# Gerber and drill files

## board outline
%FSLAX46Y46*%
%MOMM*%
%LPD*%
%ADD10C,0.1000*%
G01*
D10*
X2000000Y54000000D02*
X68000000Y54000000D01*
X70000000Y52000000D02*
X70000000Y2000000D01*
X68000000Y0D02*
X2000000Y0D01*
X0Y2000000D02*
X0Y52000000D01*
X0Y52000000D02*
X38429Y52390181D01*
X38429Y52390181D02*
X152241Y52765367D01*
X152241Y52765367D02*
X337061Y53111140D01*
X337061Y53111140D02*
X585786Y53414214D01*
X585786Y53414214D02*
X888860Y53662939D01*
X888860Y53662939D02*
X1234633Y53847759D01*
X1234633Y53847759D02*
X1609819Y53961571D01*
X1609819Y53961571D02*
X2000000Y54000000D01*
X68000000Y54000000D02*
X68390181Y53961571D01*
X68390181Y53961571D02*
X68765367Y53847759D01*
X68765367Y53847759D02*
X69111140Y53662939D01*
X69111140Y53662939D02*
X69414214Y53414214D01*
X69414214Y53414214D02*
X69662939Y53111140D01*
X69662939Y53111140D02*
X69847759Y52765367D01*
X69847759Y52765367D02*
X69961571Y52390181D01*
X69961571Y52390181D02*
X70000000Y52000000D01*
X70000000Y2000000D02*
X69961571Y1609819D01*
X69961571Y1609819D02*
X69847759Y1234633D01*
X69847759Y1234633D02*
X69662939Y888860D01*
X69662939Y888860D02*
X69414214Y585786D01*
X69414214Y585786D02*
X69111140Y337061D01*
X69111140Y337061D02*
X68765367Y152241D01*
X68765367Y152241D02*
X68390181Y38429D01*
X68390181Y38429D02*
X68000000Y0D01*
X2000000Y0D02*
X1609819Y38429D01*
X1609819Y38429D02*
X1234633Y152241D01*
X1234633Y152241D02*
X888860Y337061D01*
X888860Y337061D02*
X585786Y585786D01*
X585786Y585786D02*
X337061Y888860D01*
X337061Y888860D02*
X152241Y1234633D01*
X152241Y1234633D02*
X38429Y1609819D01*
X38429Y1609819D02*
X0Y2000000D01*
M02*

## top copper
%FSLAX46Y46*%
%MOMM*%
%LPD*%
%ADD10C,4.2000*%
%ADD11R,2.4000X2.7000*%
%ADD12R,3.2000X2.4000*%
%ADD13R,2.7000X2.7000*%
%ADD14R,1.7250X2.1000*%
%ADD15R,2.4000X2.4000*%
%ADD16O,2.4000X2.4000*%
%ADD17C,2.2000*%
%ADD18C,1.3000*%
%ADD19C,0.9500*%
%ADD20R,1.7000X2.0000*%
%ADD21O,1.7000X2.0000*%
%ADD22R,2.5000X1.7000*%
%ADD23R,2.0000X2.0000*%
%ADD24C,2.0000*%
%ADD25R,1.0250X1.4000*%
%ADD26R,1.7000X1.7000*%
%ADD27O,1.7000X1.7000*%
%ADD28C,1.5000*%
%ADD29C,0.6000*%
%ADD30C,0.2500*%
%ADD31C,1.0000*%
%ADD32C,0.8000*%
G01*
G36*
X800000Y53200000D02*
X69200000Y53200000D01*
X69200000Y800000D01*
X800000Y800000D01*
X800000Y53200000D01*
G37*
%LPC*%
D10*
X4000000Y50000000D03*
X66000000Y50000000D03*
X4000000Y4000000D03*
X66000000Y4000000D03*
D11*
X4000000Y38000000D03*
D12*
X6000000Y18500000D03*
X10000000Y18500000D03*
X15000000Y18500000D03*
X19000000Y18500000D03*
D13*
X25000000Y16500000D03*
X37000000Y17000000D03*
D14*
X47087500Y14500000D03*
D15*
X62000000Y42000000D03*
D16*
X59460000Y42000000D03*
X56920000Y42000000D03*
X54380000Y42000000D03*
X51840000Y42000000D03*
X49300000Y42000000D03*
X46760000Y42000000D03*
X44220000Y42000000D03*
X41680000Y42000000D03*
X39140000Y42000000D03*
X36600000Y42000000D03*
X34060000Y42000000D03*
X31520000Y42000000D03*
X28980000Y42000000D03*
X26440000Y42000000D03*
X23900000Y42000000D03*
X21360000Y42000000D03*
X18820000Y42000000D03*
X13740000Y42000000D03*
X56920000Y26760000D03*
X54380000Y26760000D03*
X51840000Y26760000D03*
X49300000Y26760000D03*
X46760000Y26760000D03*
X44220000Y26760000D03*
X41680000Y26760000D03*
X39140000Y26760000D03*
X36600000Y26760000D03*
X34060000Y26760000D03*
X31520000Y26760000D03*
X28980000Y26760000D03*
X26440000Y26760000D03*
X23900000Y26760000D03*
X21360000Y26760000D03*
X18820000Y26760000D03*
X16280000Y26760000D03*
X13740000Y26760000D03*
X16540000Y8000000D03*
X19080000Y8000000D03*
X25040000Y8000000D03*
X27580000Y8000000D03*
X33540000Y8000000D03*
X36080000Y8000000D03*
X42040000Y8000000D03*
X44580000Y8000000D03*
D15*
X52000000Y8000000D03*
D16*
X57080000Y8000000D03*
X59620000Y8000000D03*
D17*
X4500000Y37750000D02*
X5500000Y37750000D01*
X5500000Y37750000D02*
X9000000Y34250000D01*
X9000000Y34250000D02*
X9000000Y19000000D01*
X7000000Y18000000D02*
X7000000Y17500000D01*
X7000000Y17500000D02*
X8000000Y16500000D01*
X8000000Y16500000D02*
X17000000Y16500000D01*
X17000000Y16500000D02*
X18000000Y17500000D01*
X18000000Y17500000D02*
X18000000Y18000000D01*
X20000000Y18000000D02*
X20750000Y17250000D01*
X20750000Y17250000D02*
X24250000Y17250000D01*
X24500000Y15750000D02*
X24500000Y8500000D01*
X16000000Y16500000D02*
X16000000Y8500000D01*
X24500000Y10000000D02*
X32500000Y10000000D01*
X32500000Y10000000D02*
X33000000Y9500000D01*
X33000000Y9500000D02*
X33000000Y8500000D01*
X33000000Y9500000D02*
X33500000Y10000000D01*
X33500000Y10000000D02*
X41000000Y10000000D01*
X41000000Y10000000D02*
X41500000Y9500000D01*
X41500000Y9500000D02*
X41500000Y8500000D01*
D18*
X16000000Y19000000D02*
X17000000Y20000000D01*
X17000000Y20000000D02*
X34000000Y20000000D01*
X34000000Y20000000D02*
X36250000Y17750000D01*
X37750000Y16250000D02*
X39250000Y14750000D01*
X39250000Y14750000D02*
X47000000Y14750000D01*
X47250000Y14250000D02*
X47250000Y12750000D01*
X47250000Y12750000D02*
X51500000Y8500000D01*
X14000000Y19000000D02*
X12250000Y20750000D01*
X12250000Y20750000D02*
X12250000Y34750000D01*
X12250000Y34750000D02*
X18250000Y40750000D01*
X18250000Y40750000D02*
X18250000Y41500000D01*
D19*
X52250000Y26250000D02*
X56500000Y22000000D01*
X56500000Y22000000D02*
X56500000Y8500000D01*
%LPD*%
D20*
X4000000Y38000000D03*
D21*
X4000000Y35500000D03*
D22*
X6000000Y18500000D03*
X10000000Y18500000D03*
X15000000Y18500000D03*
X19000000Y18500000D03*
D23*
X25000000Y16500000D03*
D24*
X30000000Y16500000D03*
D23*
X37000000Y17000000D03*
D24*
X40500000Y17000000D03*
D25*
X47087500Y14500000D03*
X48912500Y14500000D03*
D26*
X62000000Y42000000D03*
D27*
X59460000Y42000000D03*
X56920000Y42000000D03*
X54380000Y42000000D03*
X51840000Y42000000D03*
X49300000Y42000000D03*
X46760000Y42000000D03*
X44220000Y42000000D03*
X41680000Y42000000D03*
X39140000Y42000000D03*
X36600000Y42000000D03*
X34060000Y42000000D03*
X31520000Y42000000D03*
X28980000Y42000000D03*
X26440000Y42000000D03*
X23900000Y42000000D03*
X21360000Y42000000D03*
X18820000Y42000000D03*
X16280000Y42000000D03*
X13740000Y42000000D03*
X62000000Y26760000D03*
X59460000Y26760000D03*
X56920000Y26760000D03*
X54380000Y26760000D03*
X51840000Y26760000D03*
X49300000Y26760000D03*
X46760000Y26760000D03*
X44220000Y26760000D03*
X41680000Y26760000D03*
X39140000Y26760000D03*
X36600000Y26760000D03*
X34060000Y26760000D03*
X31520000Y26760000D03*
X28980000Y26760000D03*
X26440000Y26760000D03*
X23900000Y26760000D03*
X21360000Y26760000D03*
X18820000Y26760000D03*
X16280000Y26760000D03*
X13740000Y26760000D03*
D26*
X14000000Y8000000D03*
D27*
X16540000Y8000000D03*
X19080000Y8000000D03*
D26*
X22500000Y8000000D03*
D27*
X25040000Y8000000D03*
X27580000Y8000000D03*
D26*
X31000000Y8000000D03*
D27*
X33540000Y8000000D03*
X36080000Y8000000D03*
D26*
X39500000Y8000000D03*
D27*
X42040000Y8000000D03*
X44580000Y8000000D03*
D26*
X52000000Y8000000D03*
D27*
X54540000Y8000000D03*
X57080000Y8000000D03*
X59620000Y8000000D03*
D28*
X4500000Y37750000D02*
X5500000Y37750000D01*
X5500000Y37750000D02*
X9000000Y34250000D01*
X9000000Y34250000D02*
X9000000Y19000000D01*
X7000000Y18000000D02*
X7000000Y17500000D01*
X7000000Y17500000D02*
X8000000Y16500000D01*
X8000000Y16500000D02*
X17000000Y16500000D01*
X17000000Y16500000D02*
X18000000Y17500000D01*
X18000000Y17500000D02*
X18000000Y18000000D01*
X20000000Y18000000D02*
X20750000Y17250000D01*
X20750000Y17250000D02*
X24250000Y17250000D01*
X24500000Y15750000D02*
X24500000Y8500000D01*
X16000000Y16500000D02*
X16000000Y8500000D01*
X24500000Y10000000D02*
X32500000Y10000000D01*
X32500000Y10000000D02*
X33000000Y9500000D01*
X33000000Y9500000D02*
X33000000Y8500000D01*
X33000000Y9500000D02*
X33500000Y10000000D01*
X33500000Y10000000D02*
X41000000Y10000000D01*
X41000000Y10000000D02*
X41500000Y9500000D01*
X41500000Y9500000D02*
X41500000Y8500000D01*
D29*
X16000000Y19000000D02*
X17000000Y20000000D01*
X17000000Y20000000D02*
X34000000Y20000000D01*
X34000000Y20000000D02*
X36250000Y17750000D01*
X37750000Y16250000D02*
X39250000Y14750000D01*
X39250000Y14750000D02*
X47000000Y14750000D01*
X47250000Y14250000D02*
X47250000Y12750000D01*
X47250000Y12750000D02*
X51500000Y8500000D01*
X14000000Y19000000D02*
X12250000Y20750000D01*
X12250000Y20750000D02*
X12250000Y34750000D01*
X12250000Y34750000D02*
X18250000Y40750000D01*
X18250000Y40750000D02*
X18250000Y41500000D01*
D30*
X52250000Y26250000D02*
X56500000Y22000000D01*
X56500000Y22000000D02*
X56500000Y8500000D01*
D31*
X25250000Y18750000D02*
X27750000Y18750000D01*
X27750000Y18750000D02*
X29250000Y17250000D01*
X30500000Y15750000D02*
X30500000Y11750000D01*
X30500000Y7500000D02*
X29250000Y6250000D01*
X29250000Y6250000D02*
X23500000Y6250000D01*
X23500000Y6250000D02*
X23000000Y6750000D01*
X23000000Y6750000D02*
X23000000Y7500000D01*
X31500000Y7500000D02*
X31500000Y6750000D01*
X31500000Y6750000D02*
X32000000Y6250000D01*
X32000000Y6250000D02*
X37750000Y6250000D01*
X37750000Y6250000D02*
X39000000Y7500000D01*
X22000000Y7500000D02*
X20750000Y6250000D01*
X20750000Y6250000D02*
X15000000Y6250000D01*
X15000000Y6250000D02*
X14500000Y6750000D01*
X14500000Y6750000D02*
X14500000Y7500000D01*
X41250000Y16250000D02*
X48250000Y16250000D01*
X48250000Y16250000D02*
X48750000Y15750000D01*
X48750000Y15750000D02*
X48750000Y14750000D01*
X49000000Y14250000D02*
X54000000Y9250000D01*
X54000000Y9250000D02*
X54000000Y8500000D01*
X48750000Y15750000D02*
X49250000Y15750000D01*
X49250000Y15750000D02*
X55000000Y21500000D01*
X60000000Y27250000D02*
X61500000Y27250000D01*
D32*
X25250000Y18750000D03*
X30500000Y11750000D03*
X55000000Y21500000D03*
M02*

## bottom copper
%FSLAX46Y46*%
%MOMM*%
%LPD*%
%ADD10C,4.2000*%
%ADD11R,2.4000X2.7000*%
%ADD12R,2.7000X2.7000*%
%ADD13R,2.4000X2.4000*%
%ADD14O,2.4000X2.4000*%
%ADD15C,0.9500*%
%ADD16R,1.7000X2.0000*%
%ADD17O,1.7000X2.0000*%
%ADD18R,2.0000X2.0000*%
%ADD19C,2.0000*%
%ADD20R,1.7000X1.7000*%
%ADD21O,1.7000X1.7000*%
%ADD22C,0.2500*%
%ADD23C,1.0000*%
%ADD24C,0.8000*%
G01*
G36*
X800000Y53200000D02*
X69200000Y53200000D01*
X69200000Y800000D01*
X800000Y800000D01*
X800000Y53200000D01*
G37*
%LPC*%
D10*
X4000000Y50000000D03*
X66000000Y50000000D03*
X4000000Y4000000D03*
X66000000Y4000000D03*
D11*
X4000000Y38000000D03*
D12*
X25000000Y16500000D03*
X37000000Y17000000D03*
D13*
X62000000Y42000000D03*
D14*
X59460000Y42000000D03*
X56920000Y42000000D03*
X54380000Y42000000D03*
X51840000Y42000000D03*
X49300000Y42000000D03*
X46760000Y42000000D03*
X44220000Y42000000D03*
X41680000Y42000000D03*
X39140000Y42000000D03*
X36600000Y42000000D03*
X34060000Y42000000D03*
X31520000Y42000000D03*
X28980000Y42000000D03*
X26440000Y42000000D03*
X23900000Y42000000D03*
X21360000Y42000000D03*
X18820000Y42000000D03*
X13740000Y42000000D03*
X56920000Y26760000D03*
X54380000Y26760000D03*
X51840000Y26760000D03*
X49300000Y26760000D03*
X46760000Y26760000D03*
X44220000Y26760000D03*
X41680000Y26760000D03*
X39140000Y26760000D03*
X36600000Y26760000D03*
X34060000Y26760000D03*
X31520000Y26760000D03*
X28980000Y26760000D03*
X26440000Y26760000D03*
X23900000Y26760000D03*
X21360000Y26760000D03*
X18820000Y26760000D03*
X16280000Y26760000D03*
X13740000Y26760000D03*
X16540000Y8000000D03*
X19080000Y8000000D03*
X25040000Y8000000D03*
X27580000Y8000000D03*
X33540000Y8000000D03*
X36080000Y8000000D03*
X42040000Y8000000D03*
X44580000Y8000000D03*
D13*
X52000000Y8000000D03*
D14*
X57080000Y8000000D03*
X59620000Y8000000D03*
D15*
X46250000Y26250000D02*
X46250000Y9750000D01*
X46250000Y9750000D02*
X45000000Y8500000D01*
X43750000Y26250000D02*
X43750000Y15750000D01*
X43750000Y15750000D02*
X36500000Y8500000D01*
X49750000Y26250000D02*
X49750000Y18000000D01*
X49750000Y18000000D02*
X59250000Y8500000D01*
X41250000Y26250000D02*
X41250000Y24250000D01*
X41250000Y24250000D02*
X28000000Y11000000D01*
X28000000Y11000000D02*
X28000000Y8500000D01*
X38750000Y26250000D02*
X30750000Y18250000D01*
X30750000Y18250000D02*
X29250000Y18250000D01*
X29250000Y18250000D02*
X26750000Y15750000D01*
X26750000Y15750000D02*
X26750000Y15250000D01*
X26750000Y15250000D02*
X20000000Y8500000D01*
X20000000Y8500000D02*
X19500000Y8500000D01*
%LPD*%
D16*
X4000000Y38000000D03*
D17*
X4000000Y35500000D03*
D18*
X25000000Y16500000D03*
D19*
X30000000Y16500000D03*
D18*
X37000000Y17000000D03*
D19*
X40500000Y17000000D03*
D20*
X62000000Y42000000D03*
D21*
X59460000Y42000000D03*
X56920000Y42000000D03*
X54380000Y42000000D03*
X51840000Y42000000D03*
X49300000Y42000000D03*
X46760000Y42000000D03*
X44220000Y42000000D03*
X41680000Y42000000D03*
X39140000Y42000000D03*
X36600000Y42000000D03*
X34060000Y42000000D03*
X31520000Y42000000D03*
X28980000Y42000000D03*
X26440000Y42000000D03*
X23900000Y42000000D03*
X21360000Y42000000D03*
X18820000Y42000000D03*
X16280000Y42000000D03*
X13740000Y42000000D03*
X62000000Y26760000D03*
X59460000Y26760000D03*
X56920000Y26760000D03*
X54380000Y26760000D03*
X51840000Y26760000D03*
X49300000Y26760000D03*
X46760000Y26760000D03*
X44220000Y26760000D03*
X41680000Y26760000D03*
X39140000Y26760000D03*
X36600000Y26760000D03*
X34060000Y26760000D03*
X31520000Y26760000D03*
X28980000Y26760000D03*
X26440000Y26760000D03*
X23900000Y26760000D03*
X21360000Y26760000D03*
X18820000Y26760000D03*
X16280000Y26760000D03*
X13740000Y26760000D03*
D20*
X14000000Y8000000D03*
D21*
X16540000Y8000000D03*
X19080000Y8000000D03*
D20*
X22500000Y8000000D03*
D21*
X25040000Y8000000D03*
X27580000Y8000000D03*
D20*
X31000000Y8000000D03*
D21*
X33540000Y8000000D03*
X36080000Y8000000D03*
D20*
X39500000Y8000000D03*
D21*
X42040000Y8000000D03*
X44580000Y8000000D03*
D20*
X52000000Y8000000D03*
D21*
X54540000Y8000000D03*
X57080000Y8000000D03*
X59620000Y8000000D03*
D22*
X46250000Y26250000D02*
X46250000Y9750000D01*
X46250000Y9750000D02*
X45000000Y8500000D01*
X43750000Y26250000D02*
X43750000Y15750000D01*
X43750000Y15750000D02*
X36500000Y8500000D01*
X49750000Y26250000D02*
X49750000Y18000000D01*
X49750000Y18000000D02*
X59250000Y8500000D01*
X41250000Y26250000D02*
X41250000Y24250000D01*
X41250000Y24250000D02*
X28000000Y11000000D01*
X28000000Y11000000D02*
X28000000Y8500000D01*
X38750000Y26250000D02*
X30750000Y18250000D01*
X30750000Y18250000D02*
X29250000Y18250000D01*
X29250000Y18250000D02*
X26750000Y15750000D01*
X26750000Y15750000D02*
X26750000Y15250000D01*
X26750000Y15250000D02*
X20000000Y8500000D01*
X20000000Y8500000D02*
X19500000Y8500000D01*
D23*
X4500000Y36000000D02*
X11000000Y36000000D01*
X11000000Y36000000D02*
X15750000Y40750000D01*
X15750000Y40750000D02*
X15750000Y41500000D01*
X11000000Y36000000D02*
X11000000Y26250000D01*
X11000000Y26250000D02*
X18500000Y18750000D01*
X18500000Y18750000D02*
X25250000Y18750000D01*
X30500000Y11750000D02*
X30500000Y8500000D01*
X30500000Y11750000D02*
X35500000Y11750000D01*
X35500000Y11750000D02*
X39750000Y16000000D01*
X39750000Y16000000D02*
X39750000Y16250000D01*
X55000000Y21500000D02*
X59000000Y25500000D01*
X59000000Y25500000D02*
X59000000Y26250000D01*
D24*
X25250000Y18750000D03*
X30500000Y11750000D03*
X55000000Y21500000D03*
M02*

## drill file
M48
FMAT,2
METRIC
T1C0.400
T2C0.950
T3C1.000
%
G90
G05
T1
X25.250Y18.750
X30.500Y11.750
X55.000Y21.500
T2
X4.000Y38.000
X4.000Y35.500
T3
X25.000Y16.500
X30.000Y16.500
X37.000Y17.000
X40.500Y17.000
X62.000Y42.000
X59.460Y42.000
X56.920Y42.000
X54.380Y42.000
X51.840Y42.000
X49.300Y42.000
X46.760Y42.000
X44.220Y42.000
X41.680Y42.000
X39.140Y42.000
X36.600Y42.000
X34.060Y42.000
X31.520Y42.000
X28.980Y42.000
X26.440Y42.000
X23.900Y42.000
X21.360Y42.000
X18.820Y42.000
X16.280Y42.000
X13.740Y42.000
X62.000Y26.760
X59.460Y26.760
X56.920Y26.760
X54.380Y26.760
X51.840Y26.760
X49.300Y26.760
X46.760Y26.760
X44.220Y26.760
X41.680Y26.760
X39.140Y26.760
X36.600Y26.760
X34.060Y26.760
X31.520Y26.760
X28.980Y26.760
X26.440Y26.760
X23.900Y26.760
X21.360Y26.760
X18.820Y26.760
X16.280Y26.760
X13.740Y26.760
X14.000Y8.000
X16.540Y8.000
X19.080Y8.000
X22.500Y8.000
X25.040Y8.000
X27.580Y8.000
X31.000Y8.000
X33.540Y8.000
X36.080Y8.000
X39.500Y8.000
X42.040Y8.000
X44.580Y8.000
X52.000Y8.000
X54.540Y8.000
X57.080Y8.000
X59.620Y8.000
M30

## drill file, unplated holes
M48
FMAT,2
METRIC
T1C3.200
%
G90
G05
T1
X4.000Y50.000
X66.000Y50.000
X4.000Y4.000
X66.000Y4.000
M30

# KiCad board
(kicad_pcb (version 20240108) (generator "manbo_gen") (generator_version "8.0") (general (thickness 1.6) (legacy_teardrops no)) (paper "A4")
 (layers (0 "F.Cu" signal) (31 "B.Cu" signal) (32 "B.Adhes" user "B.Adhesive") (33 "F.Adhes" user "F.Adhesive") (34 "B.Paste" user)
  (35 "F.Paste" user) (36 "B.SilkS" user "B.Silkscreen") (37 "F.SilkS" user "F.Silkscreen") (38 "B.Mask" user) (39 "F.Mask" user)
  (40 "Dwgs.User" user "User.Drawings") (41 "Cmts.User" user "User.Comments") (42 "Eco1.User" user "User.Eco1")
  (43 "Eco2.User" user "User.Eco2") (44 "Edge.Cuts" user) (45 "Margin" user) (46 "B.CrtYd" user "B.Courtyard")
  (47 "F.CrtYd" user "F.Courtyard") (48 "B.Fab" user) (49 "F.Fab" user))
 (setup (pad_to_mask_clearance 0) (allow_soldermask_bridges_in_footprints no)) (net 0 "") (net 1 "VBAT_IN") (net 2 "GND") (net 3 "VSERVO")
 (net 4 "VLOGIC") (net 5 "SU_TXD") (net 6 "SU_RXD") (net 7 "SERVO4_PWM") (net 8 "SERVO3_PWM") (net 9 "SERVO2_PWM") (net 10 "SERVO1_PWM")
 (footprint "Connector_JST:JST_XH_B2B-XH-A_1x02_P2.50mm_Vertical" (layer "F.Cu") (at 4 16 0)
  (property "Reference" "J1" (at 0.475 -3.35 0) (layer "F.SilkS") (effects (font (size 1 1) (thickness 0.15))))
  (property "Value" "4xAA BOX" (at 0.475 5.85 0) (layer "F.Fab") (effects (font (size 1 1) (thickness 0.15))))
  (pad "1" thru_hole roundrect (at 0 0 0) (size 1.7 2) (drill 0.95) (layers "*.Cu" "*.Mask") (roundrect_rratio 0.25) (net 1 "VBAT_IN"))
  (pad "2" thru_hole oval (at 0 2.5 0) (size 1.7 2) (drill 0.95) (layers "*.Cu" "*.Mask") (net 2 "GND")))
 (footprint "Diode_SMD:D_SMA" (layer "F.Cu") (at 8 35.5 0)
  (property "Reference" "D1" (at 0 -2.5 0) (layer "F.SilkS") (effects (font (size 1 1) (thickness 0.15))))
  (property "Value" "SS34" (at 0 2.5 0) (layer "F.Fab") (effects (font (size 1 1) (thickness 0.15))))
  (pad "1" smd rect (at -2 0 0) (size 2.5 1.7) (layers "F.Cu" "F.Paste" "F.Mask") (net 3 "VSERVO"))
  (pad "2" smd rect (at 2 0 0) (size 2.5 1.7) (layers "F.Cu" "F.Paste" "F.Mask") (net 1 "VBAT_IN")))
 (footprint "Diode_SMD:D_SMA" (layer "F.Cu") (at 17 35.5 0)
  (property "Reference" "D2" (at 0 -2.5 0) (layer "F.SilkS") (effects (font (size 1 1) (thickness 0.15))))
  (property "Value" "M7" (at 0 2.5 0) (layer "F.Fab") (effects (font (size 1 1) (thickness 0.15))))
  (pad "1" smd rect (at -2 0 0) (size 2.5 1.7) (layers "F.Cu" "F.Paste" "F.Mask") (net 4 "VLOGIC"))
  (pad "2" smd rect (at 2 0 0) (size 2.5 1.7) (layers "F.Cu" "F.Paste" "F.Mask") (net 3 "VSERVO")))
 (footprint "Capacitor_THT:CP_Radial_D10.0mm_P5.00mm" (layer "F.Cu") (at 25 37.5 0)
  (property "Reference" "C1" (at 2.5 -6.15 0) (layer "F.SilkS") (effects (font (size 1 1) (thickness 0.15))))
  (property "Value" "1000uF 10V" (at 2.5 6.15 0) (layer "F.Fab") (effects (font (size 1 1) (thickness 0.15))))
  (pad "1" thru_hole rect (at 0 0 0) (size 2 2) (drill 1) (layers "*.Cu" "*.Mask") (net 3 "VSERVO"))
  (pad "2" thru_hole circle (at 5 0 0) (size 2 2) (drill 1) (layers "*.Cu" "*.Mask") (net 2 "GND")))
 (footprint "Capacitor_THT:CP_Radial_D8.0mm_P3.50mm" (layer "F.Cu") (at 37 37 0)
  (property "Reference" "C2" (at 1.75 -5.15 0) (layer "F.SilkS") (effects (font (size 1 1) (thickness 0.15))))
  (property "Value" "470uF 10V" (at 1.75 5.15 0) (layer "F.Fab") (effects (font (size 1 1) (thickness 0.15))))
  (pad "1" thru_hole rect (at 0 0 0) (size 2 2) (drill 1) (layers "*.Cu" "*.Mask") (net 4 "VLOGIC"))
  (pad "2" thru_hole circle (at 3.5 0 0) (size 2 2) (drill 1) (layers "*.Cu" "*.Mask") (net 2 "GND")))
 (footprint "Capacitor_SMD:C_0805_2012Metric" (layer "F.Cu") (at 48 39.5 0)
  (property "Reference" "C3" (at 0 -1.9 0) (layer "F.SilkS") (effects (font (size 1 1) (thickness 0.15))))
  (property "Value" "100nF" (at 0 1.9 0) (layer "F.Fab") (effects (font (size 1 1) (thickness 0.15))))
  (pad "1" smd roundrect (at -0.9125 0 0) (size 1.025 1.4) (layers "F.Cu" "F.Paste" "F.Mask") (roundrect_rratio 0.25) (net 4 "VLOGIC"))
  (pad "2" smd roundrect (at 0.9125 0 0) (size 1.025 1.4) (layers "F.Cu" "F.Paste" "F.Mask") (roundrect_rratio 0.25) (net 2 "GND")))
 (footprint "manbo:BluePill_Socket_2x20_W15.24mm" (layer "F.Cu") (at 62 12 270)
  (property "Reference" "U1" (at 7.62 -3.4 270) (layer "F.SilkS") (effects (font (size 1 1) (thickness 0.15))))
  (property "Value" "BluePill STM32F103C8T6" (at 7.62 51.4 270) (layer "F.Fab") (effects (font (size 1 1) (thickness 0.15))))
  (pad "1" thru_hole rect (at 0 0 270) (size 1.7 1.7) (drill 1) (layers "*.Cu" "*.Mask"))
  (pad "2" thru_hole oval (at 0 2.54 270) (size 1.7 1.7) (drill 1) (layers "*.Cu" "*.Mask"))
  (pad "3" thru_hole oval (at 0 5.08 270) (size 1.7 1.7) (drill 1) (layers "*.Cu" "*.Mask"))
  (pad "4" thru_hole oval (at 0 7.62 270) (size 1.7 1.7) (drill 1) (layers "*.Cu" "*.Mask"))
  (pad "5" thru_hole oval (at 0 10.16 270) (size 1.7 1.7) (drill 1) (layers "*.Cu" "*.Mask"))
  (pad "6" thru_hole oval (at 0 12.7 270) (size 1.7 1.7) (drill 1) (layers "*.Cu" "*.Mask"))
  (pad "7" thru_hole oval (at 0 15.24 270) (size 1.7 1.7) (drill 1) (layers "*.Cu" "*.Mask"))
  (pad "8" thru_hole oval (at 0 17.78 270) (size 1.7 1.7) (drill 1) (layers "*.Cu" "*.Mask"))
  (pad "9" thru_hole oval (at 0 20.32 270) (size 1.7 1.7) (drill 1) (layers "*.Cu" "*.Mask"))
  (pad "10" thru_hole oval (at 0 22.86 270) (size 1.7 1.7) (drill 1) (layers "*.Cu" "*.Mask"))
  (pad "11" thru_hole oval (at 0 25.4 270) (size 1.7 1.7) (drill 1) (layers "*.Cu" "*.Mask"))
  (pad "12" thru_hole oval (at 0 27.94 270) (size 1.7 1.7) (drill 1) (layers "*.Cu" "*.Mask"))
  (pad "13" thru_hole oval (at 0 30.48 270) (size 1.7 1.7) (drill 1) (layers "*.Cu" "*.Mask"))
  (pad "14" thru_hole oval (at 0 33.02 270) (size 1.7 1.7) (drill 1) (layers "*.Cu" "*.Mask"))
  (pad "15" thru_hole oval (at 0 35.56 270) (size 1.7 1.7) (drill 1) (layers "*.Cu" "*.Mask"))
  (pad "16" thru_hole oval (at 0 38.1 270) (size 1.7 1.7) (drill 1) (layers "*.Cu" "*.Mask"))
  (pad "17" thru_hole oval (at 0 40.64 270) (size 1.7 1.7) (drill 1) (layers "*.Cu" "*.Mask"))
  (pad "18" thru_hole oval (at 0 43.18 270) (size 1.7 1.7) (drill 1) (layers "*.Cu" "*.Mask") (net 4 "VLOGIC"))
  (pad "19" thru_hole oval (at 0 45.72 270) (size 1.7 1.7) (drill 1) (layers "*.Cu" "*.Mask") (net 2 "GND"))
  (pad "20" thru_hole oval (at 0 48.26 270) (size 1.7 1.7) (drill 1) (layers "*.Cu" "*.Mask"))
  (pad "21" thru_hole oval (at 15.24 0 270) (size 1.7 1.7) (drill 1) (layers "*.Cu" "*.Mask") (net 2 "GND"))
  (pad "22" thru_hole oval (at 15.24 2.54 270) (size 1.7 1.7) (drill 1) (layers "*.Cu" "*.Mask") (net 2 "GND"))
  (pad "23" thru_hole oval (at 15.24 5.08 270) (size 1.7 1.7) (drill 1) (layers "*.Cu" "*.Mask"))
  (pad "24" thru_hole oval (at 15.24 7.62 270) (size 1.7 1.7) (drill 1) (layers "*.Cu" "*.Mask"))
  (pad "25" thru_hole oval (at 15.24 10.16 270) (size 1.7 1.7) (drill 1) (layers "*.Cu" "*.Mask") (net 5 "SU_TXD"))
  (pad "26" thru_hole oval (at 15.24 12.7 270) (size 1.7 1.7) (drill 1) (layers "*.Cu" "*.Mask") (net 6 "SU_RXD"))
  (pad "27" thru_hole oval (at 15.24 15.24 270) (size 1.7 1.7) (drill 1) (layers "*.Cu" "*.Mask") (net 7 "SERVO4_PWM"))
  (pad "28" thru_hole oval (at 15.24 17.78 270) (size 1.7 1.7) (drill 1) (layers "*.Cu" "*.Mask") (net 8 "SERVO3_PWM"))
  (pad "29" thru_hole oval (at 15.24 20.32 270) (size 1.7 1.7) (drill 1) (layers "*.Cu" "*.Mask") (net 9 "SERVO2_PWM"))
  (pad "30" thru_hole oval (at 15.24 22.86 270) (size 1.7 1.7) (drill 1) (layers "*.Cu" "*.Mask") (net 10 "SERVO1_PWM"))
  (pad "31" thru_hole oval (at 15.24 25.4 270) (size 1.7 1.7) (drill 1) (layers "*.Cu" "*.Mask"))
  (pad "32" thru_hole oval (at 15.24 27.94 270) (size 1.7 1.7) (drill 1) (layers "*.Cu" "*.Mask"))
  (pad "33" thru_hole oval (at 15.24 30.48 270) (size 1.7 1.7) (drill 1) (layers "*.Cu" "*.Mask"))
  (pad "34" thru_hole oval (at 15.24 33.02 270) (size 1.7 1.7) (drill 1) (layers "*.Cu" "*.Mask"))
  (pad "35" thru_hole oval (at 15.24 35.56 270) (size 1.7 1.7) (drill 1) (layers "*.Cu" "*.Mask"))
  (pad "36" thru_hole oval (at 15.24 38.1 270) (size 1.7 1.7) (drill 1) (layers "*.Cu" "*.Mask"))
  (pad "37" thru_hole oval (at 15.24 40.64 270) (size 1.7 1.7) (drill 1) (layers "*.Cu" "*.Mask"))
  (pad "38" thru_hole oval (at 15.24 43.18 270) (size 1.7 1.7) (drill 1) (layers "*.Cu" "*.Mask"))
  (pad "39" thru_hole oval (at 15.24 45.72 270) (size 1.7 1.7) (drill 1) (layers "*.Cu" "*.Mask"))
  (pad "40" thru_hole oval (at 15.24 48.26 270) (size 1.7 1.7) (drill 1) (layers "*.Cu" "*.Mask")))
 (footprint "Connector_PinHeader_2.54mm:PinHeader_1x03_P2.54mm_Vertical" (layer "F.Cu") (at 14 46 90)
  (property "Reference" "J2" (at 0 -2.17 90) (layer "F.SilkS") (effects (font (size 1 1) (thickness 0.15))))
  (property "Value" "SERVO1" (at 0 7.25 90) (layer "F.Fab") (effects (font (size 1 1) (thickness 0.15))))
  (pad "1" thru_hole rect (at 0 0 90) (size 1.7 1.7) (drill 1) (layers "*.Cu" "*.Mask") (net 2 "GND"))
  (pad "2" thru_hole oval (at 0 2.54 90) (size 1.7 1.7) (drill 1) (layers "*.Cu" "*.Mask") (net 3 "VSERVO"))
  (pad "3" thru_hole oval (at 0 5.08 90) (size 1.7 1.7) (drill 1) (layers "*.Cu" "*.Mask") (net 10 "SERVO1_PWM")))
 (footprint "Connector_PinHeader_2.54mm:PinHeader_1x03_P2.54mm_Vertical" (layer "F.Cu") (at 22.5 46 90)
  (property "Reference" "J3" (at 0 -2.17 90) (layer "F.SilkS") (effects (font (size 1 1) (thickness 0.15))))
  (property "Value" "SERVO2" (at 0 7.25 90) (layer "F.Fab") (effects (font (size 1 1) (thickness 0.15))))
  (pad "1" thru_hole rect (at 0 0 90) (size 1.7 1.7) (drill 1) (layers "*.Cu" "*.Mask") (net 2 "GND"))
  (pad "2" thru_hole oval (at 0 2.54 90) (size 1.7 1.7) (drill 1) (layers "*.Cu" "*.Mask") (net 3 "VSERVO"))
  (pad "3" thru_hole oval (at 0 5.08 90) (size 1.7 1.7) (drill 1) (layers "*.Cu" "*.Mask") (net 9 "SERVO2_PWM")))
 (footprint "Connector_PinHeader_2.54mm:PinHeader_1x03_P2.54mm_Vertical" (layer "F.Cu") (at 31 46 90)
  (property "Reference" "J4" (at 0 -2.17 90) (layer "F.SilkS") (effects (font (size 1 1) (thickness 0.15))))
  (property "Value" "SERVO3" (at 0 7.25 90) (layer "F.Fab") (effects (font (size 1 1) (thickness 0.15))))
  (pad "1" thru_hole rect (at 0 0 90) (size 1.7 1.7) (drill 1) (layers "*.Cu" "*.Mask") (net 2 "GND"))
  (pad "2" thru_hole oval (at 0 2.54 90) (size 1.7 1.7) (drill 1) (layers "*.Cu" "*.Mask") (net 3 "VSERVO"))
  (pad "3" thru_hole oval (at 0 5.08 90) (size 1.7 1.7) (drill 1) (layers "*.Cu" "*.Mask") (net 8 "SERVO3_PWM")))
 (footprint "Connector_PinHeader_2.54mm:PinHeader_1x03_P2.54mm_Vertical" (layer "F.Cu") (at 39.5 46 90)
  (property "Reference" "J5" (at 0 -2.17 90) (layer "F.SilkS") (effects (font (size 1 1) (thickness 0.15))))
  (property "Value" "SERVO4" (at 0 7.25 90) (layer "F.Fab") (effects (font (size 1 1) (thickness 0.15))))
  (pad "1" thru_hole rect (at 0 0 90) (size 1.7 1.7) (drill 1) (layers "*.Cu" "*.Mask") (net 2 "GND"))
  (pad "2" thru_hole oval (at 0 2.54 90) (size 1.7 1.7) (drill 1) (layers "*.Cu" "*.Mask") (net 3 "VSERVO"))
  (pad "3" thru_hole oval (at 0 5.08 90) (size 1.7 1.7) (drill 1) (layers "*.Cu" "*.Mask") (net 7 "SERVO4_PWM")))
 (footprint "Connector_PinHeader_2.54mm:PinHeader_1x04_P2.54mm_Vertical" (layer "F.Cu") (at 52 46 90)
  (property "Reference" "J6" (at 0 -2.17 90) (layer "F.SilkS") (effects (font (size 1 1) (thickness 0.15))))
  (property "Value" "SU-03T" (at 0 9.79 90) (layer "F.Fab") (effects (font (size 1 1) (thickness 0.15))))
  (pad "1" thru_hole rect (at 0 0 90) (size 1.7 1.7) (drill 1) (layers "*.Cu" "*.Mask") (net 4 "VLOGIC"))
  (pad "2" thru_hole oval (at 0 2.54 90) (size 1.7 1.7) (drill 1) (layers "*.Cu" "*.Mask") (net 2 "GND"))
  (pad "3" thru_hole oval (at 0 5.08 90) (size 1.7 1.7) (drill 1) (layers "*.Cu" "*.Mask") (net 5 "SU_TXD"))
  (pad "4" thru_hole oval (at 0 7.62 90) (size 1.7 1.7) (drill 1) (layers "*.Cu" "*.Mask") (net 6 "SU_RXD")))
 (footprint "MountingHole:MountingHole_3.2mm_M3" (layer "F.Cu") (at 4 4 0)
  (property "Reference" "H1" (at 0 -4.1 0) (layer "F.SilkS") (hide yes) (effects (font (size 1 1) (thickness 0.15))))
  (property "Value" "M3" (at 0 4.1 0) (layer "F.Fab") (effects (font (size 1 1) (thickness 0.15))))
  (pad "" np_thru_hole circle (at 0 0 0) (size 3.2 3.2) (drill 3.2) (layers "*.Cu" "*.Mask")))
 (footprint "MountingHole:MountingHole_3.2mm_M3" (layer "F.Cu") (at 66 4 0)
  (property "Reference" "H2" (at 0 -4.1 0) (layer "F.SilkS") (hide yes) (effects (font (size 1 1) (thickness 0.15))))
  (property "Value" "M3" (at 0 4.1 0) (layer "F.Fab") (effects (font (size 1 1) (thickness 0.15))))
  (pad "" np_thru_hole circle (at 0 0 0) (size 3.2 3.2) (drill 3.2) (layers "*.Cu" "*.Mask")))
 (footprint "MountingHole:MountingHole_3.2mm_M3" (layer "F.Cu") (at 4 50 0)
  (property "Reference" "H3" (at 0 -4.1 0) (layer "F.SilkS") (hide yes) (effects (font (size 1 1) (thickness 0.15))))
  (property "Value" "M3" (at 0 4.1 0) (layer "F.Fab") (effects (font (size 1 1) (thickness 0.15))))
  (pad "" np_thru_hole circle (at 0 0 0) (size 3.2 3.2) (drill 3.2) (layers "*.Cu" "*.Mask")))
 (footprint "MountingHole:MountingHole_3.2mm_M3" (layer "F.Cu") (at 66 50 0)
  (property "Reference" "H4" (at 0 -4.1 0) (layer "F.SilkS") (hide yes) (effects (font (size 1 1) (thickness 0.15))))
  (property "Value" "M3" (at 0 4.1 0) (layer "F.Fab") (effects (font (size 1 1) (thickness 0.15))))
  (pad "" np_thru_hole circle (at 0 0 0) (size 3.2 3.2) (drill 3.2) (layers "*.Cu" "*.Mask")))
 (gr_line (start 2 0) (end 68 0) (stroke (width 0.1) (type default)) (layer "Edge.Cuts"))
 (gr_line (start 70 2) (end 70 52) (stroke (width 0.1) (type default)) (layer "Edge.Cuts"))
 (gr_line (start 68 54) (end 2 54) (stroke (width 0.1) (type default)) (layer "Edge.Cuts"))
 (gr_line (start 0 52) (end 0 2) (stroke (width 0.1) (type default)) (layer "Edge.Cuts"))
 (gr_arc (start 0 2) (mid 0.5858 0.5858) (end 2 0) (stroke (width 0.1) (type default)) (layer "Edge.Cuts"))
 (gr_arc (start 68 0) (mid 69.4142 0.5858) (end 70 2) (stroke (width 0.1) (type default)) (layer "Edge.Cuts"))
 (gr_arc (start 70 52) (mid 69.4142 53.4142) (end 68 54) (stroke (width 0.1) (type default)) (layer "Edge.Cuts"))
 (gr_arc (start 2 54) (mid 0.5858 53.4142) (end 0 52) (stroke (width 0.1) (type default)) (layer "Edge.Cuts"))
 (segment (start 4.5 16.25) (end 5.5 16.25) (width 1.5) (layer "F.Cu") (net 1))
 (segment (start 5.5 16.25) (end 9 19.75) (width 1.5) (layer "F.Cu") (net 1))
 (segment (start 9 19.75) (end 9 35) (width 1.5) (layer "F.Cu") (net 1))
 (segment (start 7 36) (end 7 36.5) (width 1.5) (layer "F.Cu") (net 3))
 (segment (start 7 36.5) (end 8 37.5) (width 1.5) (layer "F.Cu") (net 3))
 (segment (start 8 37.5) (end 17 37.5) (width 1.5) (layer "F.Cu") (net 3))
 (segment (start 17 37.5) (end 18 36.5) (width 1.5) (layer "F.Cu") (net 3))
 (segment (start 18 36.5) (end 18 36) (width 1.5) (layer "F.Cu") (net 3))
 (segment (start 20 36) (end 20.75 36.75) (width 1.5) (layer "F.Cu") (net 3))
 (segment (start 20.75 36.75) (end 24.25 36.75) (width 1.5) (layer "F.Cu") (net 3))
 (segment (start 24.5 38.25) (end 24.5 45.5) (width 1.5) (layer "F.Cu") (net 3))
 (segment (start 16 37.5) (end 16 45.5) (width 1.5) (layer "F.Cu") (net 3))
 (segment (start 24.5 44) (end 32.5 44) (width 1.5) (layer "F.Cu") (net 3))
 (segment (start 32.5 44) (end 33 44.5) (width 1.5) (layer "F.Cu") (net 3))
 (segment (start 33 44.5) (end 33 45.5) (width 1.5) (layer "F.Cu") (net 3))
 (segment (start 33 44.5) (end 33.5 44) (width 1.5) (layer "F.Cu") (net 3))
 (segment (start 33.5 44) (end 41 44) (width 1.5) (layer "F.Cu") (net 3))
 (segment (start 41 44) (end 41.5 44.5) (width 1.5) (layer "F.Cu") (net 3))
 (segment (start 41.5 44.5) (end 41.5 45.5) (width 1.5) (layer "F.Cu") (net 3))
 (segment (start 16 35) (end 17 34) (width 0.6) (layer "F.Cu") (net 4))
 (segment (start 17 34) (end 34 34) (width 0.6) (layer "F.Cu") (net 4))
 (segment (start 34 34) (end 36.25 36.25) (width 0.6) (layer "F.Cu") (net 4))
 (segment (start 37.75 37.75) (end 39.25 39.25) (width 0.6) (layer "F.Cu") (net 4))
 (segment (start 39.25 39.25) (end 47 39.25) (width 0.6) (layer "F.Cu") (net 4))
 (segment (start 47.25 39.75) (end 47.25 41.25) (width 0.6) (layer "F.Cu") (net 4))
 (segment (start 47.25 41.25) (end 51.5 45.5) (width 0.6) (layer "F.Cu") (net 4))
 (segment (start 14 35) (end 12.25 33.25) (width 0.6) (layer "F.Cu") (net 4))
 (segment (start 12.25 33.25) (end 12.25 19.25) (width 0.6) (layer "F.Cu") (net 4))
 (segment (start 12.25 19.25) (end 18.25 13.25) (width 0.6) (layer "F.Cu") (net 4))
 (segment (start 18.25 13.25) (end 18.25 12.5) (width 0.6) (layer "F.Cu") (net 4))
 (segment (start 46.25 27.75) (end 46.25 44.25) (width 0.25) (layer "B.Cu") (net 7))
 (segment (start 46.25 44.25) (end 45 45.5) (width 0.25) (layer "B.Cu") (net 7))
 (segment (start 52.25 27.75) (end 56.5 32) (width 0.25) (layer "F.Cu") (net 5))
 (segment (start 56.5 32) (end 56.5 45.5) (width 0.25) (layer "F.Cu") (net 5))
 (segment (start 43.75 27.75) (end 43.75 38.25) (width 0.25) (layer "B.Cu") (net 8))
 (segment (start 43.75 38.25) (end 36.5 45.5) (width 0.25) (layer "B.Cu") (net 8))
 (segment (start 49.75 27.75) (end 49.75 36) (width 0.25) (layer "B.Cu") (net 6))
 (segment (start 49.75 36) (end 59.25 45.5) (width 0.25) (layer "B.Cu") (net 6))
 (segment (start 41.25 27.75) (end 41.25 29.75) (width 0.25) (layer "B.Cu") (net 9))
 (segment (start 41.25 29.75) (end 28 43) (width 0.25) (layer "B.Cu") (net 9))
 (segment (start 28 43) (end 28 45.5) (width 0.25) (layer "B.Cu") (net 9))
 (segment (start 38.75 27.75) (end 30.75 35.75) (width 0.25) (layer "B.Cu") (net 10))
 (segment (start 30.75 35.75) (end 29.25 35.75) (width 0.25) (layer "B.Cu") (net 10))
 (segment (start 29.25 35.75) (end 26.75 38.25) (width 0.25) (layer "B.Cu") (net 10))
 (segment (start 26.75 38.25) (end 26.75 38.75) (width 0.25) (layer "B.Cu") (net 10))
 (segment (start 26.75 38.75) (end 20 45.5) (width 0.25) (layer "B.Cu") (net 10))
 (segment (start 20 45.5) (end 19.5 45.5) (width 0.25) (layer "B.Cu") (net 10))
 (segment (start 4.5 18) (end 11 18) (width 1) (layer "B.Cu") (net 2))
 (segment (start 11 18) (end 15.75 13.25) (width 1) (layer "B.Cu") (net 2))
 (segment (start 15.75 13.25) (end 15.75 12.5) (width 1) (layer "B.Cu") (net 2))
 (segment (start 11 18) (end 11 27.75) (width 1) (layer "B.Cu") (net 2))
 (segment (start 11 27.75) (end 18.5 35.25) (width 1) (layer "B.Cu") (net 2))
 (segment (start 18.5 35.25) (end 25.25 35.25) (width 1) (layer "B.Cu") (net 2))
 (segment (start 25.25 35.25) (end 27.75 35.25) (width 1) (layer "F.Cu") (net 2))
 (segment (start 27.75 35.25) (end 29.25 36.75) (width 1) (layer "F.Cu") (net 2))
 (segment (start 30.5 38.25) (end 30.5 42.25) (width 1) (layer "F.Cu") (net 2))
 (segment (start 30.5 42.25) (end 30.5 45.5) (width 1) (layer "B.Cu") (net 2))
 (segment (start 30.5 46.5) (end 29.25 47.75) (width 1) (layer "F.Cu") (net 2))
 (segment (start 29.25 47.75) (end 23.5 47.75) (width 1) (layer "F.Cu") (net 2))
 (segment (start 23.5 47.75) (end 23 47.25) (width 1) (layer "F.Cu") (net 2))
 (segment (start 23 47.25) (end 23 46.5) (width 1) (layer "F.Cu") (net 2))
 (segment (start 31.5 46.5) (end 31.5 47.25) (width 1) (layer "F.Cu") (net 2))
 (segment (start 31.5 47.25) (end 32 47.75) (width 1) (layer "F.Cu") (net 2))
 (segment (start 32 47.75) (end 37.75 47.75) (width 1) (layer "F.Cu") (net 2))
 (segment (start 37.75 47.75) (end 39 46.5) (width 1) (layer "F.Cu") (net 2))
 (segment (start 22 46.5) (end 20.75 47.75) (width 1) (layer "F.Cu") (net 2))
 (segment (start 20.75 47.75) (end 15 47.75) (width 1) (layer "F.Cu") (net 2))
 (segment (start 15 47.75) (end 14.5 47.25) (width 1) (layer "F.Cu") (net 2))
 (segment (start 14.5 47.25) (end 14.5 46.5) (width 1) (layer "F.Cu") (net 2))
 (segment (start 30.5 42.25) (end 35.5 42.25) (width 1) (layer "B.Cu") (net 2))
 (segment (start 35.5 42.25) (end 39.75 38) (width 1) (layer "B.Cu") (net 2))
 (segment (start 39.75 38) (end 39.75 37.75) (width 1) (layer "B.Cu") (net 2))
 (segment (start 41.25 37.75) (end 48.25 37.75) (width 1) (layer "F.Cu") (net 2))
 (segment (start 48.25 37.75) (end 48.75 38.25) (width 1) (layer "F.Cu") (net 2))
 (segment (start 48.75 38.25) (end 48.75 39.25) (width 1) (layer "F.Cu") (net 2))
 (segment (start 49 39.75) (end 54 44.75) (width 1) (layer "F.Cu") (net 2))
 (segment (start 54 44.75) (end 54 45.5) (width 1) (layer "F.Cu") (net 2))
 (segment (start 48.75 38.25) (end 49.25 38.25) (width 1) (layer "F.Cu") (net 2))
 (segment (start 49.25 38.25) (end 55 32.5) (width 1) (layer "F.Cu") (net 2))
 (segment (start 55 32.5) (end 59 28.5) (width 1) (layer "B.Cu") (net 2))
 (segment (start 59 28.5) (end 59 27.75) (width 1) (layer "B.Cu") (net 2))
 (segment (start 60 26.75) (end 61.5 26.75) (width 1) (layer "F.Cu") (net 2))
 (via (at 25.25 35.25) (size 0.8) (drill 0.4) (layers "F.Cu" "B.Cu") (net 2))
 (via (at 30.5 42.25) (size 0.8) (drill 0.4) (layers "F.Cu" "B.Cu") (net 2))
 (via (at 55 32.5) (size 0.8) (drill 0.4) (layers "F.Cu" "B.Cu") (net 2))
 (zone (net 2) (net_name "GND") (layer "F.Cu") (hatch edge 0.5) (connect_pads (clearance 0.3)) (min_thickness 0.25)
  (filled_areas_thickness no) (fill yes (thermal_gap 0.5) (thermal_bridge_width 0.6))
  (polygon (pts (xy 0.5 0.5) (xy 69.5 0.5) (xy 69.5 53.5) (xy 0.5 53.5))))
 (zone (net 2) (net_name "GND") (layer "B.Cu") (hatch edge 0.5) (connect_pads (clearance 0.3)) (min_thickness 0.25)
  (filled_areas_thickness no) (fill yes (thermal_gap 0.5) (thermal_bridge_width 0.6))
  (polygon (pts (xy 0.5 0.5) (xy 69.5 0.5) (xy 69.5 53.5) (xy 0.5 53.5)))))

